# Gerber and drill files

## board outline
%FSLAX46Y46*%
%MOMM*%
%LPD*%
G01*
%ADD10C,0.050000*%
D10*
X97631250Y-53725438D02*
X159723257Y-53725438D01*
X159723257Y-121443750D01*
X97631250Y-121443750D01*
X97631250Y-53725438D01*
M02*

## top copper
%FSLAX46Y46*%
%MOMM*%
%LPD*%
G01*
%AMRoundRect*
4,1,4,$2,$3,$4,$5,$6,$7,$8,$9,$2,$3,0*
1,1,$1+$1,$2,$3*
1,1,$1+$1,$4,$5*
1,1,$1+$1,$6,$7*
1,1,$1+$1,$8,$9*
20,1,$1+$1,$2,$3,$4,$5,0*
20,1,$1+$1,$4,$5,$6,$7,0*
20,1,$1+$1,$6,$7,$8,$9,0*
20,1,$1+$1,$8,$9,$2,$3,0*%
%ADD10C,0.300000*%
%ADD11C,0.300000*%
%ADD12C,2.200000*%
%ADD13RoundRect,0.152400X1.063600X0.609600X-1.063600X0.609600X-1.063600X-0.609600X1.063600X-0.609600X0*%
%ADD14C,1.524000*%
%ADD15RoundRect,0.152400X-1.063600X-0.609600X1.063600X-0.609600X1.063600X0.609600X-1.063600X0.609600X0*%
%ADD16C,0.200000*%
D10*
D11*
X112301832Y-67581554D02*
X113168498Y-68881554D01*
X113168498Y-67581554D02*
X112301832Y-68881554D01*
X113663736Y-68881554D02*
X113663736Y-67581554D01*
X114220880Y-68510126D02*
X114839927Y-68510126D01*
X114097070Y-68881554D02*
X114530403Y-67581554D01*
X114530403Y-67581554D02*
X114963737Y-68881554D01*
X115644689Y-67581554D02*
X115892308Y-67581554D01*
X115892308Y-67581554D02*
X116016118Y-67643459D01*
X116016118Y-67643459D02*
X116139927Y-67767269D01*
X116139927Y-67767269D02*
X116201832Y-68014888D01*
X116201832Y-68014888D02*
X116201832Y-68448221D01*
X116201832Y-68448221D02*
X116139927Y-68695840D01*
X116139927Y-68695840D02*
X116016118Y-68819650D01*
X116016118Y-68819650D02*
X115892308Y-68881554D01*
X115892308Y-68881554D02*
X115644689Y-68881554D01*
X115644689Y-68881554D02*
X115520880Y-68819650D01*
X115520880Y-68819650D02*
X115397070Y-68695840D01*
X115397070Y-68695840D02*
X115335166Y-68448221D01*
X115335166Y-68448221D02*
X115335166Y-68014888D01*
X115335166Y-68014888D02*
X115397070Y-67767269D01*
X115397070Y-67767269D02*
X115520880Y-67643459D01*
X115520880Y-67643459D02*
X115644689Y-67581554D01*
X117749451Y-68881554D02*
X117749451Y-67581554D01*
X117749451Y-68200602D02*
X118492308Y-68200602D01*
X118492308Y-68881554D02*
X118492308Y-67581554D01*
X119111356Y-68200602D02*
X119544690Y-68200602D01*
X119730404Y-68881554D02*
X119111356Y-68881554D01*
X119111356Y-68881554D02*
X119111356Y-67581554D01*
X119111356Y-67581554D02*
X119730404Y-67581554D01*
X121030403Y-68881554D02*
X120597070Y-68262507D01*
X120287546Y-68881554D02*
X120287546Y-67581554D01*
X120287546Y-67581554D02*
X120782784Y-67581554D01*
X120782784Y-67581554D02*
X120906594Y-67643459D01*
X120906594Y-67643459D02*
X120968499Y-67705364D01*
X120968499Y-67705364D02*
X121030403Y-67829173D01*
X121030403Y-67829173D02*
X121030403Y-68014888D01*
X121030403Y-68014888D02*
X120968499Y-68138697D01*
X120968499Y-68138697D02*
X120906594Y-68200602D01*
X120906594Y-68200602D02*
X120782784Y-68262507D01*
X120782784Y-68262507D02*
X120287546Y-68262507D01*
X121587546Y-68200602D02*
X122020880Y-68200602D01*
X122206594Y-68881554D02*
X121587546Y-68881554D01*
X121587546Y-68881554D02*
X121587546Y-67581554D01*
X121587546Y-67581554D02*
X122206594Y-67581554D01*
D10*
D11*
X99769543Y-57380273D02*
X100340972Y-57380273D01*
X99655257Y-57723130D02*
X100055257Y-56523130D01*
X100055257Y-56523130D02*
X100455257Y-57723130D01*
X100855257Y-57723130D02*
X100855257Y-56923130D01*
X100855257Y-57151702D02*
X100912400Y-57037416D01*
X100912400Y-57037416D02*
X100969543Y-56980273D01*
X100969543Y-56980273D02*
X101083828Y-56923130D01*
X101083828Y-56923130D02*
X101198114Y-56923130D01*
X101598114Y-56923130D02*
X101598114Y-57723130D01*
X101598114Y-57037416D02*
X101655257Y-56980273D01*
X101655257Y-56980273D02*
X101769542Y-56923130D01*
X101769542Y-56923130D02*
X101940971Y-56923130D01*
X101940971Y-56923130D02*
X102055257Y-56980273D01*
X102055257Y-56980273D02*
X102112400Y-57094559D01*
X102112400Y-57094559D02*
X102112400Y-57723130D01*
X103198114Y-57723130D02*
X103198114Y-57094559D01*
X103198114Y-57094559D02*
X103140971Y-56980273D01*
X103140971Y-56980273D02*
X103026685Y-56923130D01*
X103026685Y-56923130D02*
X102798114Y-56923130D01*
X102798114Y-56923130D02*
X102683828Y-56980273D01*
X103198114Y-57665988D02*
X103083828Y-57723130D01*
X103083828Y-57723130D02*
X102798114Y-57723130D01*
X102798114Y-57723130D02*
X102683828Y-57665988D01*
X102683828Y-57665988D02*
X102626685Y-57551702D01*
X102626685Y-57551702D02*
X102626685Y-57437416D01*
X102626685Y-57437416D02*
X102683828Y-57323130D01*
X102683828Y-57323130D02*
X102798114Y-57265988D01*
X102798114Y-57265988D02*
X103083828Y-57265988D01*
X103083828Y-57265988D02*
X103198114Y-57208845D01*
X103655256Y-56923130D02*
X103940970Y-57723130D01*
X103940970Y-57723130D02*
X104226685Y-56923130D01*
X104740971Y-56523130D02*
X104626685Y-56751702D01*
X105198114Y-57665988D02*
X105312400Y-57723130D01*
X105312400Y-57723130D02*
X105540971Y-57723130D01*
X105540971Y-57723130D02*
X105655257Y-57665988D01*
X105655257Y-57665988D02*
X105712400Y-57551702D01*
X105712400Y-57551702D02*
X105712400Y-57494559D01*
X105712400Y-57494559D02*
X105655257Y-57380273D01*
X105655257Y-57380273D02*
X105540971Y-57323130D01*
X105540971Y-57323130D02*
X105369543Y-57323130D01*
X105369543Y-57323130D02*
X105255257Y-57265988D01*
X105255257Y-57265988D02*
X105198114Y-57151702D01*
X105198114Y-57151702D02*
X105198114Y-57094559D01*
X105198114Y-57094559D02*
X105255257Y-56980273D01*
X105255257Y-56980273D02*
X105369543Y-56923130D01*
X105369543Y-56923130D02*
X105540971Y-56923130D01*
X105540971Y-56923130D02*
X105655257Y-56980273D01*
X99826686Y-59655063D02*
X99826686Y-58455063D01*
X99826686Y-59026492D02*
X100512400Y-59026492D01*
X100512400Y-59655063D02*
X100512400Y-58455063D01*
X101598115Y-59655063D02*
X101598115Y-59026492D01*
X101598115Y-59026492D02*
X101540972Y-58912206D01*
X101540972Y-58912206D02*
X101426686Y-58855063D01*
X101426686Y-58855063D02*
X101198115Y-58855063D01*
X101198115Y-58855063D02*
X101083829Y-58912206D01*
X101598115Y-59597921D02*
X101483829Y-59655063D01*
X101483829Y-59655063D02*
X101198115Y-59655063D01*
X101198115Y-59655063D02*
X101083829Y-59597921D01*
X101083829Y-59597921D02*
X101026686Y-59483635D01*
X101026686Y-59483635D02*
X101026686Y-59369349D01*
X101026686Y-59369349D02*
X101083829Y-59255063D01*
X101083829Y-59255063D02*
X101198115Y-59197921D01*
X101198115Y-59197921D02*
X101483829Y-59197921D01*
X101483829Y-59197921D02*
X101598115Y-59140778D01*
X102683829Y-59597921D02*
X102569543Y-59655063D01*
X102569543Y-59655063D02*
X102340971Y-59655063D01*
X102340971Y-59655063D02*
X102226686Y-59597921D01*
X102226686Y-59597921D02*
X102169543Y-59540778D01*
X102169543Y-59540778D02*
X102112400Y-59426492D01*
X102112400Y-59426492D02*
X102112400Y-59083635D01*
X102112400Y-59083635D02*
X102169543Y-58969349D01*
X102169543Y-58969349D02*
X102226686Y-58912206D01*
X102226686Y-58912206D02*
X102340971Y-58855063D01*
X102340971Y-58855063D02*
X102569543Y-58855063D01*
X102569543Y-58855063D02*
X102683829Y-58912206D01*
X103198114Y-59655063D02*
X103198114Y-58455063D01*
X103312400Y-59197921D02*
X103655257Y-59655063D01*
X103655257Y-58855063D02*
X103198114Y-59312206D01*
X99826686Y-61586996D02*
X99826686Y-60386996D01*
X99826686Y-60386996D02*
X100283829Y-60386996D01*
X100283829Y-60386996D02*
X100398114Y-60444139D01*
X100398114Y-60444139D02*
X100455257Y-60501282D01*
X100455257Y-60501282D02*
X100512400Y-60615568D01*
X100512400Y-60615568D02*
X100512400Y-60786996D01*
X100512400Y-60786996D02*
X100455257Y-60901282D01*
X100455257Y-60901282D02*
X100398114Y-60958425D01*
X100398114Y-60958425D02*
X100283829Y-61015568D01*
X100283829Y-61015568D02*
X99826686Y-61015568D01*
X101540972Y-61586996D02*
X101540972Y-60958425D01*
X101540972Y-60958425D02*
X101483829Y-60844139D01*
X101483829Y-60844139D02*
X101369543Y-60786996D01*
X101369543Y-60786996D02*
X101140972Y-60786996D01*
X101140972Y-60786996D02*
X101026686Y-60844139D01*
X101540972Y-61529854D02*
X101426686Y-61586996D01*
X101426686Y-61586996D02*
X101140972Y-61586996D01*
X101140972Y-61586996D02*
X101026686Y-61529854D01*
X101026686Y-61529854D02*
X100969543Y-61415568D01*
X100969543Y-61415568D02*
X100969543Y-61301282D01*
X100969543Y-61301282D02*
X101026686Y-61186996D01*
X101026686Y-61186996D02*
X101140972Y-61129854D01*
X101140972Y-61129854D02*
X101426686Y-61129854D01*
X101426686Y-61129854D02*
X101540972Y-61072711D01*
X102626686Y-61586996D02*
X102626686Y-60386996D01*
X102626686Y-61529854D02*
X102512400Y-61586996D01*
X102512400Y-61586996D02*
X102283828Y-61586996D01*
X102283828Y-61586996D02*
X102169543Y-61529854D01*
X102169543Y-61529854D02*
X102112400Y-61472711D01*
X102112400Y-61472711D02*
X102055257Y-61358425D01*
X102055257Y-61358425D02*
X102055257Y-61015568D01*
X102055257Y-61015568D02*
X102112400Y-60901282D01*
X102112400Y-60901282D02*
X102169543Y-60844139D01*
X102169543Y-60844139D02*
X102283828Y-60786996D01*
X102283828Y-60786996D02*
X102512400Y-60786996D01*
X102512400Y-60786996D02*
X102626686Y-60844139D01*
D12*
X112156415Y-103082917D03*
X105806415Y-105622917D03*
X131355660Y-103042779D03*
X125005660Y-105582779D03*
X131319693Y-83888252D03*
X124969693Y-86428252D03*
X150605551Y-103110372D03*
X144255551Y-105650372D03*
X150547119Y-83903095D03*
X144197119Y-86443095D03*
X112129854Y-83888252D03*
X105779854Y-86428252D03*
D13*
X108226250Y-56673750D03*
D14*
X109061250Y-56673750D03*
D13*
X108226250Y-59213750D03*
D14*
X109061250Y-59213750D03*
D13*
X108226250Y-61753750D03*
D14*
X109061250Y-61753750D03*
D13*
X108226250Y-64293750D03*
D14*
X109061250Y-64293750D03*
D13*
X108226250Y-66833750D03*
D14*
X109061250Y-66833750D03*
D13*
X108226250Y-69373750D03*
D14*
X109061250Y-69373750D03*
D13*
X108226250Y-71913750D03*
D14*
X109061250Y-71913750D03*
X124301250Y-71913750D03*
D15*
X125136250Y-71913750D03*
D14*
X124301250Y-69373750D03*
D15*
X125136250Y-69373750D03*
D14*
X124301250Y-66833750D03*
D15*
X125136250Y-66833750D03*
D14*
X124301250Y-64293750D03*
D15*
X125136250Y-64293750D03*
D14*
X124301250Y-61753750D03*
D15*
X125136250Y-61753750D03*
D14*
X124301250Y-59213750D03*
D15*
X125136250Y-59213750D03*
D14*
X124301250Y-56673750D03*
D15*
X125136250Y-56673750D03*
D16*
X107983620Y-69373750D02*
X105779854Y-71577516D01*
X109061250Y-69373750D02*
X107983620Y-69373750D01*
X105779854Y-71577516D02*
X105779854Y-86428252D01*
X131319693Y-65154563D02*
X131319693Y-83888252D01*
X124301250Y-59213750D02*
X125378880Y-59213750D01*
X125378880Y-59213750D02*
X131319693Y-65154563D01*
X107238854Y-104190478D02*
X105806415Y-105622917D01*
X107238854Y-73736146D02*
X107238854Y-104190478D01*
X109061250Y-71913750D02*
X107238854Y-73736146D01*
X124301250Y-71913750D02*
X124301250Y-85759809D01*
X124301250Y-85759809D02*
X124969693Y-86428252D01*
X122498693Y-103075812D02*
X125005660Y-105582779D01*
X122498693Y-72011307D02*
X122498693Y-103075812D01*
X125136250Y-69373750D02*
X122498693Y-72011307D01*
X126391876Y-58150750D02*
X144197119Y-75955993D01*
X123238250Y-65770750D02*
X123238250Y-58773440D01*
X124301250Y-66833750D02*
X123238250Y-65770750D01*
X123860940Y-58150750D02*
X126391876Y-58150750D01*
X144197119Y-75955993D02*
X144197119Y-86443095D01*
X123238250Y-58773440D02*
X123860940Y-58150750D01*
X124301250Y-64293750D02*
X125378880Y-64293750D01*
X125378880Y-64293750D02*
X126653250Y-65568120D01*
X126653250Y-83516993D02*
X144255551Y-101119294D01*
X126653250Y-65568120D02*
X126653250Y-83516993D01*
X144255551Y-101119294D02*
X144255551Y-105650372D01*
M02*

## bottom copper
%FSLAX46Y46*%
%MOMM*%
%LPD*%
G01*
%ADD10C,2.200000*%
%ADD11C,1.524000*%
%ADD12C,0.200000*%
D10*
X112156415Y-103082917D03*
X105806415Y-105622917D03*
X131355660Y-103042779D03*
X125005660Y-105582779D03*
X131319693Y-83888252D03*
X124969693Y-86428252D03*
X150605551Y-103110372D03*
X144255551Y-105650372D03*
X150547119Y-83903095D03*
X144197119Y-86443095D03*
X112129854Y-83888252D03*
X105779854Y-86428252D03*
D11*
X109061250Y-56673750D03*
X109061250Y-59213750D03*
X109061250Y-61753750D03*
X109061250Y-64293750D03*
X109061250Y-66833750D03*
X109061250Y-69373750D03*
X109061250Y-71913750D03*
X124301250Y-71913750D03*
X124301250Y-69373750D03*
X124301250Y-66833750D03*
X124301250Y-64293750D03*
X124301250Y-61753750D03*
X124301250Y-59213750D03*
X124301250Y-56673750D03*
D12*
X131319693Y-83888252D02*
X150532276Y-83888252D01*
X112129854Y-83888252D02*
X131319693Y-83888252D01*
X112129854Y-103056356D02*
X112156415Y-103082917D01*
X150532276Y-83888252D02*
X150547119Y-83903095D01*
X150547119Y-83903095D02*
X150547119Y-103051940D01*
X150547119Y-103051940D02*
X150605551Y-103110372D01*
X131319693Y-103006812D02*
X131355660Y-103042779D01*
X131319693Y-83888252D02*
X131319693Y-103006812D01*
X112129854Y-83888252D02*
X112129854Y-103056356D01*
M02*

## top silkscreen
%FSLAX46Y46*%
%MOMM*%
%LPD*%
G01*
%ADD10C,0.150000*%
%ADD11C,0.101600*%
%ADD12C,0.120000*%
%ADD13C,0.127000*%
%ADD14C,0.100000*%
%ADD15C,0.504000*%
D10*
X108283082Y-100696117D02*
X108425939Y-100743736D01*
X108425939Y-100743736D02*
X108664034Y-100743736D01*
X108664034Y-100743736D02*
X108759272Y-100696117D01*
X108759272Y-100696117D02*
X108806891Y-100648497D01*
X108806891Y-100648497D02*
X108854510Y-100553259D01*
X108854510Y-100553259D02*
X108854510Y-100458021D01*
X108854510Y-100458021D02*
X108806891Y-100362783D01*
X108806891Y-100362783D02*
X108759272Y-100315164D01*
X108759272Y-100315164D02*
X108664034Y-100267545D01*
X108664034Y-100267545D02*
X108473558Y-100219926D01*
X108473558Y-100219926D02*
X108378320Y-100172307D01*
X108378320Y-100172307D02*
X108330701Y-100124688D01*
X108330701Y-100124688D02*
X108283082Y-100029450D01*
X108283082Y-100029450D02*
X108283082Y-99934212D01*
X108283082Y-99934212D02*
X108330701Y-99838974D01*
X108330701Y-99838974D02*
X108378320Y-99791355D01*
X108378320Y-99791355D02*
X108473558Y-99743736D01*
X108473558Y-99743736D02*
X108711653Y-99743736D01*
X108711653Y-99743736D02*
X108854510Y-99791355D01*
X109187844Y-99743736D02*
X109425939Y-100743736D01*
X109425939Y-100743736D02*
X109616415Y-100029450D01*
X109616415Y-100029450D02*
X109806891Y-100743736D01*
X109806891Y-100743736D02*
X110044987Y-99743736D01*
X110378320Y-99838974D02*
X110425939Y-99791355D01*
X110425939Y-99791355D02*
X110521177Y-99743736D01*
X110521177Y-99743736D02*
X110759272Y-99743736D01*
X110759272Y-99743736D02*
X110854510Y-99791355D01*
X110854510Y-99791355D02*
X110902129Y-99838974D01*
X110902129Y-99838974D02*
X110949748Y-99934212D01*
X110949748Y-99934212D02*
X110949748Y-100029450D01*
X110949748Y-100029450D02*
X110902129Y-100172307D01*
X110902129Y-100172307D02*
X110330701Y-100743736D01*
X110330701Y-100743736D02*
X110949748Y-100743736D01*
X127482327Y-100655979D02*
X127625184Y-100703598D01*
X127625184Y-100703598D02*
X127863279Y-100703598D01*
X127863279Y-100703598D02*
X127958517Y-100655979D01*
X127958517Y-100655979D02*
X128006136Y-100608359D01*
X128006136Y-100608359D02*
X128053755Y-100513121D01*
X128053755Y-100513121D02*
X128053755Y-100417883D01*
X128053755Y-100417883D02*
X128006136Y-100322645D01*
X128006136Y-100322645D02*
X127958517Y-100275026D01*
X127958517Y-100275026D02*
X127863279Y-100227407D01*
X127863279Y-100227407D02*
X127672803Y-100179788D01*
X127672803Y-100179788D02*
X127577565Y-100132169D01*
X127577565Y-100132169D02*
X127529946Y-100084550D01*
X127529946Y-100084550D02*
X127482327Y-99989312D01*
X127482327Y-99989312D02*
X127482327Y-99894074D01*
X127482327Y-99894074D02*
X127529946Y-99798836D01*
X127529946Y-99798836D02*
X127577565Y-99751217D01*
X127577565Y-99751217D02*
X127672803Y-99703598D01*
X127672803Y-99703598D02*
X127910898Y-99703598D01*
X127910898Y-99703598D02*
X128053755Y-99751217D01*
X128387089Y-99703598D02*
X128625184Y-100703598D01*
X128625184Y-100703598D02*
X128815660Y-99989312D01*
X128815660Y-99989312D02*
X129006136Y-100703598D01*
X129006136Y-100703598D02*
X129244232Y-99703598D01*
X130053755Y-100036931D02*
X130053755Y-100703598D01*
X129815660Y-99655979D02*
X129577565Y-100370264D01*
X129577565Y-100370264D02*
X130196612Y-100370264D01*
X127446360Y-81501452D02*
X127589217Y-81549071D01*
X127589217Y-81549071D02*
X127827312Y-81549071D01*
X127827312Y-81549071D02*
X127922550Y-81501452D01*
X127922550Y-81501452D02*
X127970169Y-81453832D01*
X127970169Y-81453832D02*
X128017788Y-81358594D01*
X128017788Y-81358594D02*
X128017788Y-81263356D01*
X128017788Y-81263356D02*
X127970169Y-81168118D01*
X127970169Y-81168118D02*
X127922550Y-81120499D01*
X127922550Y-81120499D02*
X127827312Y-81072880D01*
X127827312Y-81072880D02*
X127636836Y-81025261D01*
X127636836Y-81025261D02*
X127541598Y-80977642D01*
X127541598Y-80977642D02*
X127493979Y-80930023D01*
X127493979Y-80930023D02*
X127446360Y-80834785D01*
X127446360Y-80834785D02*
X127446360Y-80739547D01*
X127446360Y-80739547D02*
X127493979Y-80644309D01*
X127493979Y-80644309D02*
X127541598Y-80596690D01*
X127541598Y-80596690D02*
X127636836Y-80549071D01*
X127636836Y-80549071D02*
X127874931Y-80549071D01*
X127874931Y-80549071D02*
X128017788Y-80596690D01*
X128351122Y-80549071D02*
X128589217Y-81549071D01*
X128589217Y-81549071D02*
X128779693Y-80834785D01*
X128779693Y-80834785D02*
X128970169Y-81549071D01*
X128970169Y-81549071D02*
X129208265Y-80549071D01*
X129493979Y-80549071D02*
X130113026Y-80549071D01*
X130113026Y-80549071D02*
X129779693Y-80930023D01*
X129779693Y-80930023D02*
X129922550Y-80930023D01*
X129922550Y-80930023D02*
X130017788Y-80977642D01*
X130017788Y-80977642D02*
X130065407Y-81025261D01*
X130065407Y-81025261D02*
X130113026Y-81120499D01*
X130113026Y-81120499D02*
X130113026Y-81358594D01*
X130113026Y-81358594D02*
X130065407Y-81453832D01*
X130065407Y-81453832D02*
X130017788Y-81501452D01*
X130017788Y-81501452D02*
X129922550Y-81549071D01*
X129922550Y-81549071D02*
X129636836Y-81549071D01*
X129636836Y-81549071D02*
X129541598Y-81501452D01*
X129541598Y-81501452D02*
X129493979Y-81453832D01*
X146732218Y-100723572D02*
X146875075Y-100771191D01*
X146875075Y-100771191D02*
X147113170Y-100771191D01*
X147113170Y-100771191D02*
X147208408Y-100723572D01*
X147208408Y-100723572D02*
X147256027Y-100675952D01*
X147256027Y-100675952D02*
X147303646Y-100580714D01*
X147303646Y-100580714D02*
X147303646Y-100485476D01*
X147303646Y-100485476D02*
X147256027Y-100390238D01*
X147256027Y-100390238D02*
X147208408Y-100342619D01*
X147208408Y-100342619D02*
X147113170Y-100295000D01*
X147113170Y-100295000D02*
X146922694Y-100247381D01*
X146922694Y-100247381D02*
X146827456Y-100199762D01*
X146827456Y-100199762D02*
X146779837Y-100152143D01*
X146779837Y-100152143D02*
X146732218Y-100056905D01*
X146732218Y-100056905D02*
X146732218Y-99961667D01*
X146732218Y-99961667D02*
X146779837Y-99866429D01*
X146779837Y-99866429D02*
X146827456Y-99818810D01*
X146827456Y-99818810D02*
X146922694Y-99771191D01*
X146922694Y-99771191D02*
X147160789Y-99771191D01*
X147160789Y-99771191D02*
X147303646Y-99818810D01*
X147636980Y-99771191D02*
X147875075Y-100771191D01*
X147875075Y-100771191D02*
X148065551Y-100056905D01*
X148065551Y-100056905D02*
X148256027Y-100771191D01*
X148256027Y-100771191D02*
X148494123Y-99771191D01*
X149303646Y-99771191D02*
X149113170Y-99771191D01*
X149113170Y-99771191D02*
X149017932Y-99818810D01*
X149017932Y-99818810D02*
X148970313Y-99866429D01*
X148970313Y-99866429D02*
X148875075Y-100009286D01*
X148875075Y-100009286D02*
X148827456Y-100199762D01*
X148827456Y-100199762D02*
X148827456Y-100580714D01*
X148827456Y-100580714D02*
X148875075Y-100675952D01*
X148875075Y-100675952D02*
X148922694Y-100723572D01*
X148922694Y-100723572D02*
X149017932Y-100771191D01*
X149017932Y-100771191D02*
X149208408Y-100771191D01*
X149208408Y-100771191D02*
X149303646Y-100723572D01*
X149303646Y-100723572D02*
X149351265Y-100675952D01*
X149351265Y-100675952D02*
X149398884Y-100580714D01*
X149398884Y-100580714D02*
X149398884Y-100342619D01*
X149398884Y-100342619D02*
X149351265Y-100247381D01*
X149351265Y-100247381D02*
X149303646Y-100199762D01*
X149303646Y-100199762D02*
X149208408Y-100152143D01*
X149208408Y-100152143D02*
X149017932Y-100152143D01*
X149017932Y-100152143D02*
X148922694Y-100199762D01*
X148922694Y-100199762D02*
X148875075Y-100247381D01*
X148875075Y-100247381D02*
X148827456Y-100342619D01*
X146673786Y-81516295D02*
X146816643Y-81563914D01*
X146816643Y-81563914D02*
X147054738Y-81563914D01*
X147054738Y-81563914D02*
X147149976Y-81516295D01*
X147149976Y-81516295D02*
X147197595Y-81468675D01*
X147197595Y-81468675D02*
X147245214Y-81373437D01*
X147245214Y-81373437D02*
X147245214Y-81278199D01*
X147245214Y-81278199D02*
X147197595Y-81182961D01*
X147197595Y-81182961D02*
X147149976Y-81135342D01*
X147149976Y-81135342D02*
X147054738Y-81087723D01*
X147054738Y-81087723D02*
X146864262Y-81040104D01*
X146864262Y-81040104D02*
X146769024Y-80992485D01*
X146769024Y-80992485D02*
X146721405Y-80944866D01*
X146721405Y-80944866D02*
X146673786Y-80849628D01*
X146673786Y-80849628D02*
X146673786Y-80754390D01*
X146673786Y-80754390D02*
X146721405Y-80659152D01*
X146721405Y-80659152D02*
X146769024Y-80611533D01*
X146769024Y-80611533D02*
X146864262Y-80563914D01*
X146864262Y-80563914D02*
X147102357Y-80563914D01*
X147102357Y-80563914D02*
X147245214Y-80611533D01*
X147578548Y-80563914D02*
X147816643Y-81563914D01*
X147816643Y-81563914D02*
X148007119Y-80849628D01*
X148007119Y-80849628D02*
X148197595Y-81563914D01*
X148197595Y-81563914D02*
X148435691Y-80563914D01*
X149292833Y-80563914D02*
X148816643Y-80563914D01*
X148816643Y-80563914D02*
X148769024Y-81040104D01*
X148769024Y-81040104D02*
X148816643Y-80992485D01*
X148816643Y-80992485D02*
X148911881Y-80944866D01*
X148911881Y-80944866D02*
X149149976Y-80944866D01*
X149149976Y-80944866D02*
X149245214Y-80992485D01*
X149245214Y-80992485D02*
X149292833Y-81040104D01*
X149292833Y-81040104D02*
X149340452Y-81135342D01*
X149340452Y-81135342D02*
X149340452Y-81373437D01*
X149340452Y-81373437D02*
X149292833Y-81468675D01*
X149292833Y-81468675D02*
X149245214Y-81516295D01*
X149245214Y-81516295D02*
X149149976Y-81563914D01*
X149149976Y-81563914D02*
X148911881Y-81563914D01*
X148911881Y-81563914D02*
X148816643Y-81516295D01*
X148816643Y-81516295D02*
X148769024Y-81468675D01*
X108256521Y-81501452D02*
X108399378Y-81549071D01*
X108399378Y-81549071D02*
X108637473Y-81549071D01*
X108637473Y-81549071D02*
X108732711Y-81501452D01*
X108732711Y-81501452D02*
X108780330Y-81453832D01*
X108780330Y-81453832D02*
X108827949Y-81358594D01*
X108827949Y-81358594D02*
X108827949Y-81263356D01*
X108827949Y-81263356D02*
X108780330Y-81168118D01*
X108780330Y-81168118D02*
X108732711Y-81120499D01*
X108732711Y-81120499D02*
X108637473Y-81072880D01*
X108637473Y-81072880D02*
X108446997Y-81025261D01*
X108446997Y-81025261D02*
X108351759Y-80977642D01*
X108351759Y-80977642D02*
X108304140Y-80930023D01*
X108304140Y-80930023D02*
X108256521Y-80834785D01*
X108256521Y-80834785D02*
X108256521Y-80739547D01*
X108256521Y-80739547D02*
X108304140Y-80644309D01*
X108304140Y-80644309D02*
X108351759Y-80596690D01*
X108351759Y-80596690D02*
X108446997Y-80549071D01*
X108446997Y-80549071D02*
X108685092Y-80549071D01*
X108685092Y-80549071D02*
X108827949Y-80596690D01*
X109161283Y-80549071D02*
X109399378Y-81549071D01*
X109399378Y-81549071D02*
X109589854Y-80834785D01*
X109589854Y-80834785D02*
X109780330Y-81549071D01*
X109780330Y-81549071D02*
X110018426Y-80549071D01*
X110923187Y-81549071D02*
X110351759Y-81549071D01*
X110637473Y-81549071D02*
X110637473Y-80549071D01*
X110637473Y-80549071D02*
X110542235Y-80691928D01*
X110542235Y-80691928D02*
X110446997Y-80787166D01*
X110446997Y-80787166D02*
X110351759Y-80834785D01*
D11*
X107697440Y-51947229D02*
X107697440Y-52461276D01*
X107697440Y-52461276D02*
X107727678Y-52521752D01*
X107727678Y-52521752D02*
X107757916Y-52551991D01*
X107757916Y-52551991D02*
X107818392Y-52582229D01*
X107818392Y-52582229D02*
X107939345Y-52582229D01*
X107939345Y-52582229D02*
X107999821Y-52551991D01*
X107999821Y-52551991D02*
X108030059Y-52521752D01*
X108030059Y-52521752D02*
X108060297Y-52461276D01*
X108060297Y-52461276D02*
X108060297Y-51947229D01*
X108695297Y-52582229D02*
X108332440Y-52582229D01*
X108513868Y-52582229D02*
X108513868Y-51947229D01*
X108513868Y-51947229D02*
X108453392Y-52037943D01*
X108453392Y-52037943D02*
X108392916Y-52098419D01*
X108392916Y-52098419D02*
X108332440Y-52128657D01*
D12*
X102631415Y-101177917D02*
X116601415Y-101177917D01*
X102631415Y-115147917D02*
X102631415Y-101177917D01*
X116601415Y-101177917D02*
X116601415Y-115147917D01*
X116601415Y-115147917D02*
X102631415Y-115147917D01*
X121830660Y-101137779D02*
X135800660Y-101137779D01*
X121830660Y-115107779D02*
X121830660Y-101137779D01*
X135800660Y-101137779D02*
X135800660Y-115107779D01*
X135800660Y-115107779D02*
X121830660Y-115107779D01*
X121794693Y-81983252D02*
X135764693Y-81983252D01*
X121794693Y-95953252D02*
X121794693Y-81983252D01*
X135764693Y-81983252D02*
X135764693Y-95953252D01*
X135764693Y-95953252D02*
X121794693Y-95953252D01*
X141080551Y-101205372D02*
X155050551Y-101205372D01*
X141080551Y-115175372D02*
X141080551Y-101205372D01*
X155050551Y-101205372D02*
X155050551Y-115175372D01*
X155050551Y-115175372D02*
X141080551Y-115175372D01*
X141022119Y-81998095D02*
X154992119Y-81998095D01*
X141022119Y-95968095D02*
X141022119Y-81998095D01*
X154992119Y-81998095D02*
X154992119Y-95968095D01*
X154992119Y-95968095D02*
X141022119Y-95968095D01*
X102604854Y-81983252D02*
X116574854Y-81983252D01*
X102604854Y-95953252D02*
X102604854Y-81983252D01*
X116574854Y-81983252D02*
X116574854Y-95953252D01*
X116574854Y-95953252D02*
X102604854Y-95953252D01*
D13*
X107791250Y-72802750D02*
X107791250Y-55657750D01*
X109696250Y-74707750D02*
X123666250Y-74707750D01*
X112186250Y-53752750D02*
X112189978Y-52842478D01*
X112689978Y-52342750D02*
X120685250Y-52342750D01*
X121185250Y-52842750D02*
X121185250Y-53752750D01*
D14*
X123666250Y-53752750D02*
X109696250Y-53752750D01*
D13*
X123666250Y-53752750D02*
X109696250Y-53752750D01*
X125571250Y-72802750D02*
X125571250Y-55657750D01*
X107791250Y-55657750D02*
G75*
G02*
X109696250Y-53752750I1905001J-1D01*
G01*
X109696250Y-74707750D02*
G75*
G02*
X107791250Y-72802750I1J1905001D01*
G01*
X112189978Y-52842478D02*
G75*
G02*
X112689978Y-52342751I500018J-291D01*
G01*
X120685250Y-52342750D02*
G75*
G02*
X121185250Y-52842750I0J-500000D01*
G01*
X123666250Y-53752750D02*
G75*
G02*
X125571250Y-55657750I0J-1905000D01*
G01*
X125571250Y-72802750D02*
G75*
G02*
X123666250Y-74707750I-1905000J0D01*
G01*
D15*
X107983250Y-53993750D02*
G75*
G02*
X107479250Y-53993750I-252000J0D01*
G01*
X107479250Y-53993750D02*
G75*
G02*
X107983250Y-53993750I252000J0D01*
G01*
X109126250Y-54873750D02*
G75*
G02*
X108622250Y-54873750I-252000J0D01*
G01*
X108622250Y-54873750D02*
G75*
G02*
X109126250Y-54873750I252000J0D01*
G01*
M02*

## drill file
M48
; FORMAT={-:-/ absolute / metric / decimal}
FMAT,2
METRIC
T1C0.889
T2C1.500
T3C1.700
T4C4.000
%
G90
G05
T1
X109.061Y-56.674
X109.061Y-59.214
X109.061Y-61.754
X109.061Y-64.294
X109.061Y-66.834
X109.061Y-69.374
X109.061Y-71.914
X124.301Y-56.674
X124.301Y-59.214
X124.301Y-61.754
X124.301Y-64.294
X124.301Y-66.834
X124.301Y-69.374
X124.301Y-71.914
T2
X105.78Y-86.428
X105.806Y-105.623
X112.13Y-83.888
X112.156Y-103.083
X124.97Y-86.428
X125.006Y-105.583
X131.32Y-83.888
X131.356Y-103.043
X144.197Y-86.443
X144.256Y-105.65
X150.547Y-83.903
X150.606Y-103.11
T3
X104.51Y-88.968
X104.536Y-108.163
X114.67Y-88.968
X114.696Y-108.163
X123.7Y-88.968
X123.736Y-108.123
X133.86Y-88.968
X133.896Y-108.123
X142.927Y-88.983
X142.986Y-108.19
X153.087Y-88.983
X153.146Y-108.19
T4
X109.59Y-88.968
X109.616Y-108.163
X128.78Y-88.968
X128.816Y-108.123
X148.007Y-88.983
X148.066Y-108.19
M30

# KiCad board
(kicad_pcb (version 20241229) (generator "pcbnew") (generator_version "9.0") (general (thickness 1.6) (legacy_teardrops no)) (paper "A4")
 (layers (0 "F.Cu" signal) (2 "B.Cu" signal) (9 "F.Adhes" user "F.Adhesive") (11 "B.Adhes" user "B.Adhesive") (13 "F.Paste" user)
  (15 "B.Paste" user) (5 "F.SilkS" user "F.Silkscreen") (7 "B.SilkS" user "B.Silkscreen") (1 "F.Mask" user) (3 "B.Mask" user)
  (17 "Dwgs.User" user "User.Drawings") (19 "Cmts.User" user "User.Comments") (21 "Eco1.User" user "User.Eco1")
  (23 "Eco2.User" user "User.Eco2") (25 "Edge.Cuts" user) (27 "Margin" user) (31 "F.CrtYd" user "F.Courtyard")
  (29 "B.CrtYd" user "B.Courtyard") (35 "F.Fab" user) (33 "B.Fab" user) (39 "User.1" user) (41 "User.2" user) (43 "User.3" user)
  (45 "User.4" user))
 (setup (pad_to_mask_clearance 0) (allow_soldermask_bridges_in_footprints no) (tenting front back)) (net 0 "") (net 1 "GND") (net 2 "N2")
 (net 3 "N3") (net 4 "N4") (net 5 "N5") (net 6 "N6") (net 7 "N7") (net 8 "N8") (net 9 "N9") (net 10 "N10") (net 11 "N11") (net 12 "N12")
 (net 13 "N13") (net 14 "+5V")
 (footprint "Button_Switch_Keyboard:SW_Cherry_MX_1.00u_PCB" (layer "F.Cu") (at 112.156415 103.082917)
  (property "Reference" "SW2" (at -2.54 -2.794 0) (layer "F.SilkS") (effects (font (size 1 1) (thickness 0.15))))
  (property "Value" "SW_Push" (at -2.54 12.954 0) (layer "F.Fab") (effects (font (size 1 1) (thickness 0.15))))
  (fp_line (start -9.525 -1.905) (end 4.445 -1.905) (stroke (width 0.12) (type solid)) (layer "F.SilkS"))
  (fp_line (start -9.525 12.065) (end -9.525 -1.905) (stroke (width 0.12) (type solid)) (layer "F.SilkS"))
  (fp_line (start 4.445 -1.905) (end 4.445 12.065) (stroke (width 0.12) (type solid)) (layer "F.SilkS"))
  (fp_line (start 4.445 12.065) (end -9.525 12.065) (stroke (width 0.12) (type solid)) (layer "F.SilkS"))
  (pad "" np_thru_hole circle (at -7.62 5.08) (size 1.7 1.7) (drill 1.7) (layers "*.Cu" "*.Mask"))
  (pad "" np_thru_hole circle (at -2.54 5.08) (size 4 4) (drill 4) (layers "*.Cu" "*.Mask"))
  (pad "" np_thru_hole circle (at 2.54 5.08) (size 1.7 1.7) (drill 1.7) (layers "*.Cu" "*.Mask"))
  (pad "1" thru_hole circle (at 0 0) (size 2.2 2.2) (drill 1.5) (layers "*.Cu" "*.Mask") (remove_unused_layers no) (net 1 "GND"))
  (pad "2" thru_hole circle (at -6.35 2.54) (size 2.2 2.2) (drill 1.5) (layers "*.Cu" "*.Mask") (remove_unused_layers no) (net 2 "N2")))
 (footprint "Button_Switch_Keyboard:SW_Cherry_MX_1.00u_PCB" (layer "F.Cu") (at 131.35566 103.042779)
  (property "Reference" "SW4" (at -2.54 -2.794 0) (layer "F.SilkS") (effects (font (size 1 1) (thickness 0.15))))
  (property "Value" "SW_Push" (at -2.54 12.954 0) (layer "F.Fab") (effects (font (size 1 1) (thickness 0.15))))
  (fp_line (start -9.525 -1.905) (end 4.445 -1.905) (stroke (width 0.12) (type solid)) (layer "F.SilkS"))
  (fp_line (start -9.525 12.065) (end -9.525 -1.905) (stroke (width 0.12) (type solid)) (layer "F.SilkS"))
  (fp_line (start 4.445 -1.905) (end 4.445 12.065) (stroke (width 0.12) (type solid)) (layer "F.SilkS"))
  (fp_line (start 4.445 12.065) (end -9.525 12.065) (stroke (width 0.12) (type solid)) (layer "F.SilkS"))
  (pad "" np_thru_hole circle (at -7.62 5.08) (size 1.7 1.7) (drill 1.7) (layers "*.Cu" "*.Mask"))
  (pad "" np_thru_hole circle (at -2.54 5.08) (size 4 4) (drill 4) (layers "*.Cu" "*.Mask"))
  (pad "" np_thru_hole circle (at 2.54 5.08) (size 1.7 1.7) (drill 1.7) (layers "*.Cu" "*.Mask"))
  (pad "1" thru_hole circle (at 0 0) (size 2.2 2.2) (drill 1.5) (layers "*.Cu" "*.Mask") (remove_unused_layers no) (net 1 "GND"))
  (pad "2" thru_hole circle (at -6.35 2.54) (size 2.2 2.2) (drill 1.5) (layers "*.Cu" "*.Mask") (remove_unused_layers no) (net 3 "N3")))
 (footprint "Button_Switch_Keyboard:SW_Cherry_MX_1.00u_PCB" (layer "F.Cu") (at 131.319693 83.888252)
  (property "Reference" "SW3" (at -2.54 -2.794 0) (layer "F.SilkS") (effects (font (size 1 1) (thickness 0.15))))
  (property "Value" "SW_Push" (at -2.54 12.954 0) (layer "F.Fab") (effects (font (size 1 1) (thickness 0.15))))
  (fp_line (start -9.525 -1.905) (end 4.445 -1.905) (stroke (width 0.12) (type solid)) (layer "F.SilkS"))
  (fp_line (start -9.525 12.065) (end -9.525 -1.905) (stroke (width 0.12) (type solid)) (layer "F.SilkS"))
  (fp_line (start 4.445 -1.905) (end 4.445 12.065) (stroke (width 0.12) (type solid)) (layer "F.SilkS"))
  (fp_line (start 4.445 12.065) (end -9.525 12.065) (stroke (width 0.12) (type solid)) (layer "F.SilkS"))
  (pad "" np_thru_hole circle (at -7.62 5.08) (size 1.7 1.7) (drill 1.7) (layers "*.Cu" "*.Mask"))
  (pad "" np_thru_hole circle (at -2.54 5.08) (size 4 4) (drill 4) (layers "*.Cu" "*.Mask"))
  (pad "" np_thru_hole circle (at 2.54 5.08) (size 1.7 1.7) (drill 1.7) (layers "*.Cu" "*.Mask"))
  (pad "1" thru_hole circle (at 0 0) (size 2.2 2.2) (drill 1.5) (layers "*.Cu" "*.Mask") (remove_unused_layers no) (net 1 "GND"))
  (pad "2" thru_hole circle (at -6.35 2.54) (size 2.2 2.2) (drill 1.5) (layers "*.Cu" "*.Mask") (remove_unused_layers no) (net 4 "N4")))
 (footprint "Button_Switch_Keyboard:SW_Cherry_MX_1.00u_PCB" (layer "F.Cu") (at 150.605551 103.110372)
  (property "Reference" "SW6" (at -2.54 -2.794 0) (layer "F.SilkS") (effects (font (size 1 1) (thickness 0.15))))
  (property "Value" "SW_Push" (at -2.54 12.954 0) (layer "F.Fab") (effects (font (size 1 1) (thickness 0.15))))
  (fp_line (start -9.525 -1.905) (end 4.445 -1.905) (stroke (width 0.12) (type solid)) (layer "F.SilkS"))
  (fp_line (start -9.525 12.065) (end -9.525 -1.905) (stroke (width 0.12) (type solid)) (layer "F.SilkS"))
  (fp_line (start 4.445 -1.905) (end 4.445 12.065) (stroke (width 0.12) (type solid)) (layer "F.SilkS"))
  (fp_line (start 4.445 12.065) (end -9.525 12.065) (stroke (width 0.12) (type solid)) (layer "F.SilkS"))
  (pad "" np_thru_hole circle (at -7.62 5.08) (size 1.7 1.7) (drill 1.7) (layers "*.Cu" "*.Mask"))
  (pad "" np_thru_hole circle (at -2.54 5.08) (size 4 4) (drill 4) (layers "*.Cu" "*.Mask"))
  (pad "" np_thru_hole circle (at 2.54 5.08) (size 1.7 1.7) (drill 1.7) (layers "*.Cu" "*.Mask"))
  (pad "1" thru_hole circle (at 0 0) (size 2.2 2.2) (drill 1.5) (layers "*.Cu" "*.Mask") (remove_unused_layers no) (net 1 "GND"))
  (pad "2" thru_hole circle (at -6.35 2.54) (size 2.2 2.2) (drill 1.5) (layers "*.Cu" "*.Mask") (remove_unused_layers no) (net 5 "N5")))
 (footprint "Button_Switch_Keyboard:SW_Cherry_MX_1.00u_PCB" (layer "F.Cu") (at 150.547119 83.903095)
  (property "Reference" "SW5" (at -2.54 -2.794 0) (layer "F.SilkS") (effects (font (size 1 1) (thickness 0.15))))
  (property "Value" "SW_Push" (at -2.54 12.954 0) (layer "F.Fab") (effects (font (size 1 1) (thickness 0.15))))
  (fp_line (start -9.525 -1.905) (end 4.445 -1.905) (stroke (width 0.12) (type solid)) (layer "F.SilkS"))
  (fp_line (start -9.525 12.065) (end -9.525 -1.905) (stroke (width 0.12) (type solid)) (layer "F.SilkS"))
  (fp_line (start 4.445 -1.905) (end 4.445 12.065) (stroke (width 0.12) (type solid)) (layer "F.SilkS"))
  (fp_line (start 4.445 12.065) (end -9.525 12.065) (stroke (width 0.12) (type solid)) (layer "F.SilkS"))
  (pad "" np_thru_hole circle (at -7.62 5.08) (size 1.7 1.7) (drill 1.7) (layers "*.Cu" "*.Mask"))
  (pad "" np_thru_hole circle (at -2.54 5.08) (size 4 4) (drill 4) (layers "*.Cu" "*.Mask"))
  (pad "" np_thru_hole circle (at 2.54 5.08) (size 1.7 1.7) (drill 1.7) (layers "*.Cu" "*.Mask"))
  (pad "1" thru_hole circle (at 0 0) (size 2.2 2.2) (drill 1.5) (layers "*.Cu" "*.Mask") (remove_unused_layers no) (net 1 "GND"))
  (pad "2" thru_hole circle (at -6.35 2.54) (size 2.2 2.2) (drill 1.5) (layers "*.Cu" "*.Mask") (remove_unused_layers no) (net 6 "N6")))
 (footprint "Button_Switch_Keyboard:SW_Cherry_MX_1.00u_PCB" (layer "F.Cu") (at 112.129854 83.888252)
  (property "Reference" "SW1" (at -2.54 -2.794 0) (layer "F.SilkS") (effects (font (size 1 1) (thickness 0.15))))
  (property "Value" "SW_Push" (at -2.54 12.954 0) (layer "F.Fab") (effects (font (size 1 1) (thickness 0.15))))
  (fp_line (start -9.525 -1.905) (end 4.445 -1.905) (stroke (width 0.12) (type solid)) (layer "F.SilkS"))
  (fp_line (start -9.525 12.065) (end -9.525 -1.905) (stroke (width 0.12) (type solid)) (layer "F.SilkS"))
  (fp_line (start 4.445 -1.905) (end 4.445 12.065) (stroke (width 0.12) (type solid)) (layer "F.SilkS"))
  (fp_line (start 4.445 12.065) (end -9.525 12.065) (stroke (width 0.12) (type solid)) (layer "F.SilkS"))
  (pad "" np_thru_hole circle (at -7.62 5.08) (size 1.7 1.7) (drill 1.7) (layers "*.Cu" "*.Mask"))
  (pad "" np_thru_hole circle (at -2.54 5.08) (size 4 4) (drill 4) (layers "*.Cu" "*.Mask"))
  (pad "" np_thru_hole circle (at 2.54 5.08) (size 1.7 1.7) (drill 1.7) (layers "*.Cu" "*.Mask"))
  (pad "1" thru_hole circle (at 0 0) (size 2.2 2.2) (drill 1.5) (layers "*.Cu" "*.Mask") (remove_unused_layers no) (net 1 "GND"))
  (pad "2" thru_hole circle (at -6.35 2.54) (size 2.2 2.2) (drill 1.5) (layers "*.Cu" "*.Mask") (remove_unused_layers no) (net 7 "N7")))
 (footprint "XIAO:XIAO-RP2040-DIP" (layer "F.Cu") (at 116.68125 64.29375)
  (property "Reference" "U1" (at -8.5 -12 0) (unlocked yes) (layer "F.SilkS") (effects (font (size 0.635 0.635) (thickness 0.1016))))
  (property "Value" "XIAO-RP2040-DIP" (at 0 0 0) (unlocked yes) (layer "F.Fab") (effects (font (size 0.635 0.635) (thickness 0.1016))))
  (fp_line (start -8.89 8.509) (end -8.89 -8.636) (stroke (width 0.127) (type solid)) (layer "F.SilkS"))
  (fp_line (start -6.985 10.414) (end 6.985 10.414) (stroke (width 0.127) (type solid)) (layer "F.SilkS"))
  (fp_line (start -4.495 -10.541) (end -4.491272 -11.451272) (stroke (width 0.127) (type solid)) (layer "F.SilkS"))
  (fp_line (start -3.991272 -11.951) (end 4.004 -11.951) (stroke (width 0.127) (type solid)) (layer "F.SilkS"))
  (fp_line (start 4.504 -11.451) (end 4.504 -10.541) (stroke (width 0.127) (type solid)) (layer "F.SilkS"))
  (fp_line (start 6.985 -10.541) (end -6.985 -10.541) (stroke (width 0.1) (type solid)) (layer "F.SilkS"))
  (fp_line (start 6.985 -10.541) (end -6.985 -10.541) (stroke (width 0.127) (type solid)) (layer "F.SilkS"))
  (fp_line (start 8.89 8.509) (end 8.89 -8.636) (stroke (width 0.127) (type solid)) (layer "F.SilkS"))
  (fp_arc (start -8.89 -8.636) (mid -8.332038 -9.983038) (end -6.985 -10.541) (stroke (width 0.127) (type solid)) (layer "F.SilkS"))
  (fp_arc (start -6.985 10.414) (mid -8.332038 9.856038) (end -8.89 8.509) (stroke (width 0.127) (type solid)) (layer "F.SilkS"))
  (fp_arc (start -4.491272 -11.451272) (mid -4.344728 -11.80464) (end -3.991272 -11.951) (stroke (width 0.127) (type default))
   (layer "F.SilkS"))
  (fp_arc (start 4.004 -11.951) (mid 4.357553 -11.804553) (end 4.504 -11.451) (stroke (width 0.127) (type default)) (layer "F.SilkS"))
  (fp_arc (start 6.985 -10.541) (mid 8.332038 -9.983038) (end 8.89 -8.636) (stroke (width 0.127) (type solid)) (layer "F.SilkS"))
  (fp_arc (start 8.89 8.509) (mid 8.332038 9.856038) (end 6.985 10.414) (stroke (width 0.127) (type solid)) (layer "F.SilkS"))
  (fp_circle (center -8.95 -10.3) (end -8.95 -10.554) (stroke (width 0.5) (type solid)) (fill yes) (layer "F.SilkS"))
  (fp_circle (center -7.807 -9.42) (end -7.807 -9.674) (stroke (width 0.5) (type solid)) (fill yes) (layer "F.SilkS"))
  (pad "1" smd roundrect (at -8.455 -7.62 180) (size 2.432 1.524) (layers "F.Cu" "F.Mask") (roundrect_rratio 0.1) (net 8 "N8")
   (thermal_bridge_angle 45))
  (pad "1" thru_hole circle (at -7.62 -7.62 180) (size 1.524 1.524) (drill 0.889) (layers "*.Cu" "*.Mask") (remove_unused_layers no)
   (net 8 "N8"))
  (pad "2" smd roundrect (at -8.455 -5.08 180) (size 2.432 1.524) (layers "F.Cu" "F.Mask") (roundrect_rratio 0.1) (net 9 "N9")
   (thermal_bridge_angle 45))
  (pad "2" thru_hole circle (at -7.62 -5.08 180) (size 1.524 1.524) (drill 0.889) (layers "*.Cu" "*.Mask") (remove_unused_layers no)
   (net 9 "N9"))
  (pad "3" smd roundrect (at -8.455 -2.54 180) (size 2.432 1.524) (layers "F.Cu" "F.Mask") (roundrect_rratio 0.1) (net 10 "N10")
   (thermal_bridge_angle 45))
  (pad "3" thru_hole circle (at -7.62 -2.54 180) (size 1.524 1.524) (drill 0.889) (layers "*.Cu" "*.Mask") (remove_unused_layers no)
   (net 10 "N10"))
  (pad "4" smd roundrect (at -8.455 0 180) (size 2.432 1.524) (layers "F.Cu" "F.Mask") (roundrect_rratio 0.1) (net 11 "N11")
   (thermal_bridge_angle 45))
  (pad "4" thru_hole circle (at -7.62 0 180) (size 1.524 1.524) (drill 0.889) (layers "*.Cu" "*.Mask") (remove_unused_layers no)
   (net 11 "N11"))
  (pad "5" smd roundrect (at -8.455 2.54 180) (size 2.432 1.524) (layers "F.Cu" "F.Mask") (roundrect_rratio 0.1) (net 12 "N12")
   (thermal_bridge_angle 45))
  (pad "5" thru_hole circle (at -7.62 2.54 180) (size 1.524 1.524) (drill 0.889) (layers "*.Cu" "*.Mask") (remove_unused_layers no)
   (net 12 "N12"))
  (pad "6" smd roundrect (at -8.455 5.08 180) (size 2.432 1.524) (layers "F.Cu" "F.Mask") (roundrect_rratio 0.1) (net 7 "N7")
   (thermal_bridge_angle 45))
  (pad "6" thru_hole circle (at -7.62 5.08 180) (size 1.524 1.524) (drill 0.889) (layers "*.Cu" "*.Mask") (remove_unused_layers no)
   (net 7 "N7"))
  (pad "7" smd roundrect (at -8.455 7.62 180) (size 2.432 1.524) (layers "F.Cu" "F.Mask") (roundrect_rratio 0.1) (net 2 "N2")
   (thermal_bridge_angle 45))
  (pad "7" thru_hole circle (at -7.62 7.62 180) (size 1.524 1.524) (drill 0.889) (layers "*.Cu" "*.Mask") (remove_unused_layers no)
   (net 2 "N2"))
  (pad "8" thru_hole circle (at 7.62 7.62) (size 1.524 1.524) (drill 0.889) (layers "*.Cu" "*.Mask") (remove_unused_layers no) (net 4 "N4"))
  (pad "8" smd roundrect (at 8.455 7.62) (size 2.432 1.524) (layers "F.Cu" "F.Mask") (roundrect_rratio 0.1) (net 4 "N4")
   (thermal_bridge_angle 45))
  (pad "9" thru_hole circle (at 7.62 5.08) (size 1.524 1.524) (drill 0.889) (layers "*.Cu" "*.Mask") (remove_unused_layers no) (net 3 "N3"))
  (pad "9" smd roundrect (at 8.455 5.08) (size 2.432 1.524) (layers "F.Cu" "F.Mask") (roundrect_rratio 0.1) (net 3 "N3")
   (thermal_bridge_angle 45))
  (pad "10" thru_hole circle (at 7.62 2.54) (size 1.524 1.524) (drill 0.889) (layers "*.Cu" "*.Mask") (remove_unused_layers no) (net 6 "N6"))
  (pad "10" smd roundrect (at 8.455 2.54) (size 2.432 1.524) (layers "F.Cu" "F.Mask") (roundrect_rratio 0.1) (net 6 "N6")
   (thermal_bridge_angle 45))
  (pad "11" thru_hole circle (at 7.62 0) (size 1.524 1.524) (drill 0.889) (layers "*.Cu" "*.Mask") (remove_unused_layers no) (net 5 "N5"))
  (pad "11" smd roundrect (at 8.455 0) (size 2.432 1.524) (layers "F.Cu" "F.Mask") (roundrect_rratio 0.1) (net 5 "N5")
   (thermal_bridge_angle 45))
  (pad "12" thru_hole circle (at 7.62 -2.54) (size 1.524 1.524) (drill 0.889) (layers "*.Cu" "*.Mask") (remove_unused_layers no)
   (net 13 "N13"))
  (pad "12" smd roundrect (at 8.455 -2.54) (size 2.432 1.524) (layers "F.Cu" "F.Mask") (roundrect_rratio 0.1) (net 13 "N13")
   (thermal_bridge_angle 45))
  (pad "13" thru_hole circle (at 7.62 -5.08) (size 1.524 1.524) (drill 0.889) (layers "*.Cu" "*.Mask") (remove_unused_layers no)
   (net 1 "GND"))
  (pad "13" smd roundrect (at 8.455 -5.08) (size 2.432 1.524) (layers "F.Cu" "F.Mask") (roundrect_rratio 0.1) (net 1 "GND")
   (thermal_bridge_angle 45))
  (pad "14" thru_hole circle (at 7.62 -7.62) (size 1.524 1.524) (drill 0.889) (layers "*.Cu" "*.Mask") (remove_unused_layers no)
   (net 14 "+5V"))
  (pad "14" smd roundrect (at 8.455 -7.62) (size 2.432 1.524) (layers "F.Cu" "F.Mask") (roundrect_rratio 0.1) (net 14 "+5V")
   (thermal_bridge_angle 45)))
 (gr_rect (start 97.63125 53.725438) (end 159.723257 121.44375) (stroke (width 0.05) (type default)) (fill no) (layer "Edge.Cuts"))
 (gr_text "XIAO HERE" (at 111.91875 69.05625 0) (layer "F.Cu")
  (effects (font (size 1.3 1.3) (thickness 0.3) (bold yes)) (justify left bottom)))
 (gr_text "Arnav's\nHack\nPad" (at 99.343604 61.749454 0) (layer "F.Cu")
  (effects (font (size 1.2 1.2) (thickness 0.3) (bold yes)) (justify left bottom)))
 (segment (start 107.98362 69.37375) (end 105.779854 71.577516) (width 0.2) (layer "F.Cu") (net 7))
 (segment (start 109.06125 69.37375) (end 107.98362 69.37375) (width 0.2) (layer "F.Cu") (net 7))
 (segment (start 105.779854 71.577516) (end 105.779854 86.428252) (width 0.2) (layer "F.Cu") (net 7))
 (segment (start 131.319693 65.154563) (end 131.319693 83.888252) (width 0.2) (layer "F.Cu") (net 1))
 (segment (start 124.30125 59.21375) (end 125.37888 59.21375) (width 0.2) (layer "F.Cu") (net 1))
 (segment (start 125.37888 59.21375) (end 131.319693 65.154563) (width 0.2) (layer "F.Cu") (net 1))
 (segment (start 131.319693 83.888252) (end 150.532276 83.888252) (width 0.2) (layer "B.Cu") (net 1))
 (segment (start 112.129854 83.888252) (end 131.319693 83.888252) (width 0.2) (layer "B.Cu") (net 1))
 (segment (start 112.129854 103.056356) (end 112.156415 103.082917) (width 0.2) (layer "B.Cu") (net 1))
 (segment (start 150.532276 83.888252) (end 150.547119 83.903095) (width 0.2) (layer "B.Cu") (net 1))
 (segment (start 150.547119 83.903095) (end 150.547119 103.05194) (width 0.2) (layer "B.Cu") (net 1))
 (segment (start 150.547119 103.05194) (end 150.605551 103.110372) (width 0.2) (layer "B.Cu") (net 1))
 (segment (start 131.319693 103.006812) (end 131.35566 103.042779) (width 0.2) (layer "B.Cu") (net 1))
 (segment (start 131.319693 83.888252) (end 131.319693 103.006812) (width 0.2) (layer "B.Cu") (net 1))
 (segment (start 112.129854 83.888252) (end 112.129854 103.056356) (width 0.2) (layer "B.Cu") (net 1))
 (segment (start 107.238854 104.190478) (end 105.806415 105.622917) (width 0.2) (layer "F.Cu") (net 2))
 (segment (start 107.238854 73.736146) (end 107.238854 104.190478) (width 0.2) (layer "F.Cu") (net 2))
 (segment (start 109.06125 71.91375) (end 107.238854 73.736146) (width 0.2) (layer "F.Cu") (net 2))
 (segment (start 124.30125 71.91375) (end 124.30125 85.759809) (width 0.2) (layer "F.Cu") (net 4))
 (segment (start 124.30125 85.759809) (end 124.969693 86.428252) (width 0.2) (layer "F.Cu") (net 4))
 (segment (start 122.498693 103.075812) (end 125.00566 105.582779) (width 0.2) (layer "F.Cu") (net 3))
 (segment (start 122.498693 72.011307) (end 122.498693 103.075812) (width 0.2) (layer "F.Cu") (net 3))
 (segment (start 125.13625 69.37375) (end 122.498693 72.011307) (width 0.2) (layer "F.Cu") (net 3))
 (segment (start 126.391876 58.15075) (end 144.197119 75.955993) (width 0.2) (layer "F.Cu") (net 6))
 (segment (start 123.23825 65.77075) (end 123.23825 58.77344) (width 0.2) (layer "F.Cu") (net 6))
 (segment (start 124.30125 66.83375) (end 123.23825 65.77075) (width 0.2) (layer "F.Cu") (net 6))
 (segment (start 123.86094 58.15075) (end 126.391876 58.15075) (width 0.2) (layer "F.Cu") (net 6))
 (segment (start 144.197119 75.955993) (end 144.197119 86.443095) (width 0.2) (layer "F.Cu") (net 6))
 (segment (start 123.23825 58.77344) (end 123.86094 58.15075) (width 0.2) (layer "F.Cu") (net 6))
 (segment (start 124.30125 64.29375) (end 125.37888 64.29375) (width 0.2) (layer "F.Cu") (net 5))
 (segment (start 125.37888 64.29375) (end 126.65325 65.56812) (width 0.2) (layer "F.Cu") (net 5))
 (segment (start 126.65325 83.516993) (end 144.255551 101.119294) (width 0.2) (layer "F.Cu") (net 5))
 (segment (start 126.65325 65.56812) (end 126.65325 83.516993) (width 0.2) (layer "F.Cu") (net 5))
 (segment (start 144.255551 101.119294) (end 144.255551 105.650372) (width 0.2) (layer "F.Cu") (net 5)))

